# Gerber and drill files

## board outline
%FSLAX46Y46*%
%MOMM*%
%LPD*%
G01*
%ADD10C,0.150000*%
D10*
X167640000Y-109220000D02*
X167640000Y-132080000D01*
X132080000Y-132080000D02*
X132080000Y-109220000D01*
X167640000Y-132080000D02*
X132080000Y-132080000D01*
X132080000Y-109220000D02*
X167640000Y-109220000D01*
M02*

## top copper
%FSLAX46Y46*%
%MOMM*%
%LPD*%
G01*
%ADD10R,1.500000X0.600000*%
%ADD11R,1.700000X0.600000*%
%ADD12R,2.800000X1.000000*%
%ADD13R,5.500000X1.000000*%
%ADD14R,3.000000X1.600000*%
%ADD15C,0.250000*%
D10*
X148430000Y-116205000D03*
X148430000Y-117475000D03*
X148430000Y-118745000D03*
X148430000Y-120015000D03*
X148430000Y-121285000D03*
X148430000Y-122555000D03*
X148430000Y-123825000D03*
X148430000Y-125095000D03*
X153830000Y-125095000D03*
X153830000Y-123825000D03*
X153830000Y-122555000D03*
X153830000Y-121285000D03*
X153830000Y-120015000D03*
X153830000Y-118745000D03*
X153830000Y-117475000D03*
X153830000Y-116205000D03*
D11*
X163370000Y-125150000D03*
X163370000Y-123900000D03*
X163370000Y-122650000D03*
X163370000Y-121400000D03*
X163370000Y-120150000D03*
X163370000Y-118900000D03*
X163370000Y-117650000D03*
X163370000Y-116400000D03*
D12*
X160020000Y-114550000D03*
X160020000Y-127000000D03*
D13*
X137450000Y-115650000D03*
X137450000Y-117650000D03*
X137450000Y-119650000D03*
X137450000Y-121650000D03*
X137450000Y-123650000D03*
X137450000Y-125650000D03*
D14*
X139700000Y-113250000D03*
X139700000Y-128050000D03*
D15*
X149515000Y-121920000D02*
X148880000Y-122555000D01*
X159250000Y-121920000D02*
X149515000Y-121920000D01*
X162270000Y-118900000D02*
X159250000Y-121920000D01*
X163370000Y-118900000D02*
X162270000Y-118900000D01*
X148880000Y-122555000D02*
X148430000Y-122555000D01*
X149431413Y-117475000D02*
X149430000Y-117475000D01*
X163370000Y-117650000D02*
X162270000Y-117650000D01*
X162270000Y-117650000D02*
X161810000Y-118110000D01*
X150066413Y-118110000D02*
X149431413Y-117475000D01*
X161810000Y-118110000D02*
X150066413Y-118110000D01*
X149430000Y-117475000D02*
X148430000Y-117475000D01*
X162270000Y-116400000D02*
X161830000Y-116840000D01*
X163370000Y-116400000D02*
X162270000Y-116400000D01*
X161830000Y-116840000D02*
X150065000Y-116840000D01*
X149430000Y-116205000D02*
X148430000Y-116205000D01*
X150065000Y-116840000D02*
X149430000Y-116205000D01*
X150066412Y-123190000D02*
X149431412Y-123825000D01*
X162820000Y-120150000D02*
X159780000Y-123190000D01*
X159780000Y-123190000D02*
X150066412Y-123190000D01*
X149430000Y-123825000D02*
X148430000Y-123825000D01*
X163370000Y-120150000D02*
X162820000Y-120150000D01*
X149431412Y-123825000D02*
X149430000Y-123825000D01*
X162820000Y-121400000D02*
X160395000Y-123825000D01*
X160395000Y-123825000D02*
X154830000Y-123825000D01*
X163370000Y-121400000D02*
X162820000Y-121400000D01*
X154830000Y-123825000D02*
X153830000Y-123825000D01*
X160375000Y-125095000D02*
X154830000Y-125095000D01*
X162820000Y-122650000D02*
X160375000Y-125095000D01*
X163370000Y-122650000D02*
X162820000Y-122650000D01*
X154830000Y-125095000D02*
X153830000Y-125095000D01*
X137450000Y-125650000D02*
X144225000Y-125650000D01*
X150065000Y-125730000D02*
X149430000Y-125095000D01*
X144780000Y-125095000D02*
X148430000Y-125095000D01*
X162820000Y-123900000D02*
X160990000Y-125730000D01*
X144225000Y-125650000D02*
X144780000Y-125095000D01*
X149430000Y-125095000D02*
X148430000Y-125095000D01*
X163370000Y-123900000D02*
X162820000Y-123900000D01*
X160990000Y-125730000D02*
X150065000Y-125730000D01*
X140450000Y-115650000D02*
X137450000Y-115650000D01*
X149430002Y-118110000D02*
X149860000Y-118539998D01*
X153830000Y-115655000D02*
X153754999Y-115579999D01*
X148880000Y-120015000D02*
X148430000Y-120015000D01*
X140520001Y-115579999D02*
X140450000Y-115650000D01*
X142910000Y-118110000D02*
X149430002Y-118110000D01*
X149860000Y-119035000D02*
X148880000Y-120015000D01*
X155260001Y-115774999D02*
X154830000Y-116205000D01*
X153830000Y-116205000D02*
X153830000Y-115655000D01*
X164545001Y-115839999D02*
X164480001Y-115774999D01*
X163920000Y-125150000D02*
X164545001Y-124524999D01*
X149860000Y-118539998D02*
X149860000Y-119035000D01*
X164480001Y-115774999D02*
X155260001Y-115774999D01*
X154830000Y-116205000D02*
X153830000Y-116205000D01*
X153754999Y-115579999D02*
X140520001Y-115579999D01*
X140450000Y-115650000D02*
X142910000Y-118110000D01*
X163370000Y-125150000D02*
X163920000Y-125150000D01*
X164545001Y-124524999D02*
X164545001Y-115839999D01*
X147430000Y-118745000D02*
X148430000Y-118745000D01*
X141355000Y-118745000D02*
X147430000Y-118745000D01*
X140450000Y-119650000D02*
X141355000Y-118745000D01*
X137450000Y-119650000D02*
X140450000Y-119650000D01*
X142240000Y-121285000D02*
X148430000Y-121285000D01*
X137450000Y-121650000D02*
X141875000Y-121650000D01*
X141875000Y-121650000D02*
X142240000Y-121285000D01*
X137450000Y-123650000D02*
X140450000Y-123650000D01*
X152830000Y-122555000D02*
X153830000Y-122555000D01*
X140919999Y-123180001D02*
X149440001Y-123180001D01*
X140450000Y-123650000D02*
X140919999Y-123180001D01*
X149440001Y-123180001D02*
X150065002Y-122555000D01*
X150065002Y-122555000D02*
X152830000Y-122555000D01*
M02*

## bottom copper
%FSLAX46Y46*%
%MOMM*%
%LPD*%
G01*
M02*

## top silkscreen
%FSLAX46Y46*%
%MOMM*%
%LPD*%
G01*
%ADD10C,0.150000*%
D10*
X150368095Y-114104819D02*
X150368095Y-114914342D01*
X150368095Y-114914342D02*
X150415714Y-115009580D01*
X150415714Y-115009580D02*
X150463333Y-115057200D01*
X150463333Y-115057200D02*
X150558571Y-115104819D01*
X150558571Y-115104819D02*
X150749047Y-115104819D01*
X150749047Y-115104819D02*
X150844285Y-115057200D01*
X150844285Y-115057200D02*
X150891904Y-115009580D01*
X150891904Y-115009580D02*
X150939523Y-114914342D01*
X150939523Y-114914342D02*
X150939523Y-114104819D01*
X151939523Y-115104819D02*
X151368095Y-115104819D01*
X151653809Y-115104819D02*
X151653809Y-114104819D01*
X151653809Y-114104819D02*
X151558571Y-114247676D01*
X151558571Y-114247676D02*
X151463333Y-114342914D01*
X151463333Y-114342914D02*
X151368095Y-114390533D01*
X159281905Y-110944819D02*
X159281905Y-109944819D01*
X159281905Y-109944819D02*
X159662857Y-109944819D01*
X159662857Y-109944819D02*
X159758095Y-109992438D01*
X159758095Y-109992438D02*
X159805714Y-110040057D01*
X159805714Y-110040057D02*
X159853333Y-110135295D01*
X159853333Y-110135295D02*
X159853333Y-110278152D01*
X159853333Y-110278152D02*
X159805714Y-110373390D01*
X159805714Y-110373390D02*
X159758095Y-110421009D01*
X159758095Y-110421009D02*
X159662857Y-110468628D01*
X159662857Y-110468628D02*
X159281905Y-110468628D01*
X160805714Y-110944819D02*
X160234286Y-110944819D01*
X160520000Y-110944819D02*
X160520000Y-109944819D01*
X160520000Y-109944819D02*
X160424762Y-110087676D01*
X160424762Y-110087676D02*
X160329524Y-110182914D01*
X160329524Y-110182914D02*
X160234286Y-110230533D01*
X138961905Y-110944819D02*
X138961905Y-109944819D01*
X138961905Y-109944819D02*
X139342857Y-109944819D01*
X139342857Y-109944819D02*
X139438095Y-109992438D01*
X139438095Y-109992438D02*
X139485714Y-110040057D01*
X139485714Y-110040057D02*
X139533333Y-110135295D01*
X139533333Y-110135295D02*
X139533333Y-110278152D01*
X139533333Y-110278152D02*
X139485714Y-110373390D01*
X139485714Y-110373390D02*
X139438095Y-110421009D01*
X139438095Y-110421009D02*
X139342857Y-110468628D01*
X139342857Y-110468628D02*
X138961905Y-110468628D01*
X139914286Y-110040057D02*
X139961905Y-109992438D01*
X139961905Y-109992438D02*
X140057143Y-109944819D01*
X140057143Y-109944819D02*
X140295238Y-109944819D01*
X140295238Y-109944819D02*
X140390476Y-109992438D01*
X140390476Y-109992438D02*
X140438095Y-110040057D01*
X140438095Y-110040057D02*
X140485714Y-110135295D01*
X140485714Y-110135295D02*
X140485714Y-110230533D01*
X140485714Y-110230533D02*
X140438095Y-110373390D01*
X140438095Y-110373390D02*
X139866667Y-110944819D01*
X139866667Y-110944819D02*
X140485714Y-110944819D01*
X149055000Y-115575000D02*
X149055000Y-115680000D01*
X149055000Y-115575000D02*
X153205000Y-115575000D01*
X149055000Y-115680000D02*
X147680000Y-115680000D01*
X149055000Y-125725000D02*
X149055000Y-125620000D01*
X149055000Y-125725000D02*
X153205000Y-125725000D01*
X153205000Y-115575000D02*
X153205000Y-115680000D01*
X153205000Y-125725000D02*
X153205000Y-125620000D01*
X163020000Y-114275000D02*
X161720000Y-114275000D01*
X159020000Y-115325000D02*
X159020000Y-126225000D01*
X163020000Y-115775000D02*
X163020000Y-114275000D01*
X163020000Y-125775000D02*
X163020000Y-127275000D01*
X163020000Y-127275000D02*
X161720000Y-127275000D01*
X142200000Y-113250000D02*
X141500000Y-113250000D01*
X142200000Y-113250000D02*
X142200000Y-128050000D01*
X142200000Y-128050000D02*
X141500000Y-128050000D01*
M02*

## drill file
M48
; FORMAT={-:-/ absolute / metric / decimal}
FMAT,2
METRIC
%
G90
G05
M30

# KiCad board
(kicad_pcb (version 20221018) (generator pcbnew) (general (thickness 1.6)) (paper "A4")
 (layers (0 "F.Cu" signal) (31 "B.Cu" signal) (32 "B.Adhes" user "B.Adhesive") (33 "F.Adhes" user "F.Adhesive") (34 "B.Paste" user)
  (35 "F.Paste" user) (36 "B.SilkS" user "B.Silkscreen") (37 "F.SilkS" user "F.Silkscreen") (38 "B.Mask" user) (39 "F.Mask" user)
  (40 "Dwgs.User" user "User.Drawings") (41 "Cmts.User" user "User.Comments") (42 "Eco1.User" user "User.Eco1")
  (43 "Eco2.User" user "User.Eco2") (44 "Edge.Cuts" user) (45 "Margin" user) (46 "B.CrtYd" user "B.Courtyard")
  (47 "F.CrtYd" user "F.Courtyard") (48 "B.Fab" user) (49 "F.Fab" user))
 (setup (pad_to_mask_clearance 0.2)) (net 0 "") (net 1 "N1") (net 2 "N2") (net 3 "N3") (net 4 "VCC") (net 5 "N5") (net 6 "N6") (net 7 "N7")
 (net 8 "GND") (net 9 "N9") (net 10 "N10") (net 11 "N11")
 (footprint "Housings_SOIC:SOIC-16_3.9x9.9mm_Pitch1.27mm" (layer "F.Cu") (at 151.13 120.65)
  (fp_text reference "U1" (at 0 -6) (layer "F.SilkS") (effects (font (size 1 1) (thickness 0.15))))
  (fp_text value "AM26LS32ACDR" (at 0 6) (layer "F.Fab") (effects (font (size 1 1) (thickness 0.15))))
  (fp_line (start -2.075 -5.075) (end -2.075 -4.97) (stroke (width 0.15) (type solid)) (layer "F.SilkS"))
  (fp_line (start -2.075 -5.075) (end 2.075 -5.075) (stroke (width 0.15) (type solid)) (layer "F.SilkS"))
  (fp_line (start -2.075 -4.97) (end -3.45 -4.97) (stroke (width 0.15) (type solid)) (layer "F.SilkS"))
  (fp_line (start -2.075 5.075) (end -2.075 4.97) (stroke (width 0.15) (type solid)) (layer "F.SilkS"))
  (fp_line (start -2.075 5.075) (end 2.075 5.075) (stroke (width 0.15) (type solid)) (layer "F.SilkS"))
  (fp_line (start 2.075 -5.075) (end 2.075 -4.97) (stroke (width 0.15) (type solid)) (layer "F.SilkS"))
  (fp_line (start 2.075 5.075) (end 2.075 4.97) (stroke (width 0.15) (type solid)) (layer "F.SilkS"))
  (pad "1" smd rect (at -2.7 -4.445) (size 1.5 0.6) (layers "F.Cu" "F.Paste" "F.Mask") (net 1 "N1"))
  (pad "2" smd rect (at -2.7 -3.175) (size 1.5 0.6) (layers "F.Cu" "F.Paste" "F.Mask") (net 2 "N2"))
  (pad "3" smd rect (at -2.7 -1.905) (size 1.5 0.6) (layers "F.Cu" "F.Paste" "F.Mask") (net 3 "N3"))
  (pad "4" smd rect (at -2.7 -0.635) (size 1.5 0.6) (layers "F.Cu" "F.Paste" "F.Mask") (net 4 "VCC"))
  (pad "5" smd rect (at -2.7 0.635) (size 1.5 0.6) (layers "F.Cu" "F.Paste" "F.Mask") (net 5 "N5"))
  (pad "6" smd rect (at -2.7 1.905) (size 1.5 0.6) (layers "F.Cu" "F.Paste" "F.Mask") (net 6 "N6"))
  (pad "7" smd rect (at -2.7 3.175) (size 1.5 0.6) (layers "F.Cu" "F.Paste" "F.Mask") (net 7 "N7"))
  (pad "8" smd rect (at -2.7 4.445) (size 1.5 0.6) (layers "F.Cu" "F.Paste" "F.Mask") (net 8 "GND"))
  (pad "9" smd rect (at 2.7 4.445) (size 1.5 0.6) (layers "F.Cu" "F.Paste" "F.Mask") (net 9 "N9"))
  (pad "10" smd rect (at 2.7 3.175) (size 1.5 0.6) (layers "F.Cu" "F.Paste" "F.Mask") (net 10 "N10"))
  (pad "11" smd rect (at 2.7 1.905) (size 1.5 0.6) (layers "F.Cu" "F.Paste" "F.Mask") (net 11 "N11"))
  (pad "12" smd rect (at 2.7 0.635) (size 1.5 0.6) (layers "F.Cu" "F.Paste" "F.Mask"))
  (pad "13" smd rect (at 2.7 -0.635) (size 1.5 0.6) (layers "F.Cu" "F.Paste" "F.Mask"))
  (pad "14" smd rect (at 2.7 -1.905) (size 1.5 0.6) (layers "F.Cu" "F.Paste" "F.Mask"))
  (pad "15" smd rect (at 2.7 -3.175) (size 1.5 0.6) (layers "F.Cu" "F.Paste" "F.Mask"))
  (pad "16" smd rect (at 2.7 -4.445) (size 1.5 0.6) (layers "F.Cu" "F.Paste" "F.Mask") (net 4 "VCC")))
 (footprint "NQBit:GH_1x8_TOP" (layer "F.Cu") (at 160.02 120.775 -90)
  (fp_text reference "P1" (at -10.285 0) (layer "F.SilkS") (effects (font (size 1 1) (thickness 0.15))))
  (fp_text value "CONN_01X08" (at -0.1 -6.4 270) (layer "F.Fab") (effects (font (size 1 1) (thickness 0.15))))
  (fp_line (start -6.5 -3) (end -6.5 -1.7) (stroke (width 0.15) (type solid)) (layer "F.SilkS"))
  (fp_line (start -5.45 1) (end 5.45 1) (stroke (width 0.15) (type solid)) (layer "F.SilkS"))
  (fp_line (start -5 -3) (end -6.5 -3) (stroke (width 0.15) (type solid)) (layer "F.SilkS"))
  (fp_line (start 5 -3) (end 6.5 -3) (stroke (width 0.15) (type solid)) (layer "F.SilkS"))
  (fp_line (start 6.5 -3) (end 6.5 -1.7) (stroke (width 0.15) (type solid)) (layer "F.SilkS"))
  (pad "1" smd rect (at 4.375 -3.35 270) (size 0.6 1.7) (layers "F.Cu" "F.Paste" "F.Mask") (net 4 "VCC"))
  (pad "2" smd rect (at 3.125 -3.35 270) (size 0.6 1.7) (layers "F.Cu" "F.Paste" "F.Mask") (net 8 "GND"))
  (pad "3" smd rect (at 1.875 -3.35 270) (size 0.6 1.7) (layers "F.Cu" "F.Paste" "F.Mask") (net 9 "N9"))
  (pad "4" smd rect (at 0.625 -3.35 270) (size 0.6 1.7) (layers "F.Cu" "F.Paste" "F.Mask") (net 10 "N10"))
  (pad "5" smd rect (at -0.625 -3.35 270) (size 0.6 1.7) (layers "F.Cu" "F.Paste" "F.Mask") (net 7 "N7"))
  (pad "6" smd rect (at -1.875 -3.35 270) (size 0.6 1.7) (layers "F.Cu" "F.Paste" "F.Mask") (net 6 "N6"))
  (pad "7" smd rect (at -3.125 -3.35 270) (size 0.6 1.7) (layers "F.Cu" "F.Paste" "F.Mask") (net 2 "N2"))
  (pad "8" smd rect (at -4.375 -3.35 270) (size 0.6 1.7) (layers "F.Cu" "F.Paste" "F.Mask") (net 1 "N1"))
  (pad "MECH" smd rect (at -6.225 0 270) (size 1 2.8) (layers "F.Cu" "F.Paste" "F.Mask"))
  (pad "MECH" smd rect (at 6.225 0 270) (size 1 2.8) (layers "F.Cu" "F.Paste" "F.Mask")))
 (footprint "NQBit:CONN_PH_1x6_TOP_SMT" (layer "F.Cu") (at 139.7 120.65 -90)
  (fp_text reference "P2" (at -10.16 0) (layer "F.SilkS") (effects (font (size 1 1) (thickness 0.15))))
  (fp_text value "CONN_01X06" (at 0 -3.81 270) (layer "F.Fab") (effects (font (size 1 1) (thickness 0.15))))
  (fp_line (start -7.4 -2.5) (end -7.4 -1.8) (stroke (width 0.15) (type solid)) (layer "F.SilkS"))
  (fp_line (start -7.4 -2.5) (end 7.4 -2.5) (stroke (width 0.15) (type solid)) (layer "F.SilkS"))
  (fp_line (start 7.4 -2.5) (end 7.4 -1.8) (stroke (width 0.15) (type solid)) (layer "F.SilkS"))
  (pad "1" smd rect (at -5 2.25 270) (size 1 5.5) (layers "F.Cu" "F.Paste" "F.Mask") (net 4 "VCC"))
  (pad "2" smd rect (at -3 2.25 270) (size 1 5.5) (layers "F.Cu" "F.Paste" "F.Mask"))
  (pad "3" smd rect (at -1 2.25 270) (size 1 5.5) (layers "F.Cu" "F.Paste" "F.Mask") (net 3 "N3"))
  (pad "4" smd rect (at 1 2.25 270) (size 1 5.5) (layers "F.Cu" "F.Paste" "F.Mask") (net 5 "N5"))
  (pad "5" smd rect (at 3 2.25 270) (size 1 5.5) (layers "F.Cu" "F.Paste" "F.Mask") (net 11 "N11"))
  (pad "6" smd rect (at 5 2.25 270) (size 1 5.5) (layers "F.Cu" "F.Paste" "F.Mask") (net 8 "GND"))
  (pad "MECH" smd rect (at -7.4 0 270) (size 1.6 3) (layers "F.Cu" "F.Paste" "F.Mask"))
  (pad "MECH" smd rect (at 7.4 0 270) (size 1.6 3) (layers "F.Cu" "F.Paste" "F.Mask")))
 (gr_line (start 167.64 109.22) (end 167.64 132.08) (stroke (width 0.15) (type solid)) (layer "Edge.Cuts"))
 (gr_line (start 132.08 132.08) (end 132.08 109.22) (stroke (width 0.15) (type solid)) (layer "Edge.Cuts"))
 (gr_line (start 167.64 132.08) (end 132.08 132.08) (stroke (width 0.15) (type solid)) (layer "Edge.Cuts"))
 (gr_line (start 132.08 109.22) (end 167.64 109.22) (stroke (width 0.15) (type solid)) (layer "Edge.Cuts"))
 (segment (start 149.515 121.92) (end 148.88 122.555) (width 0.25) (layer "F.Cu") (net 6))
 (segment (start 159.25 121.92) (end 149.515 121.92) (width 0.25) (layer "F.Cu") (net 6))
 (segment (start 162.27 118.9) (end 159.25 121.92) (width 0.25) (layer "F.Cu") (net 6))
 (segment (start 163.37 118.9) (end 162.27 118.9) (width 0.25) (layer "F.Cu") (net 6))
 (segment (start 148.88 122.555) (end 148.43 122.555) (width 0.25) (layer "F.Cu") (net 6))
 (segment (start 149.431413 117.475) (end 149.43 117.475) (width 0.25) (layer "F.Cu") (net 2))
 (segment (start 163.37 117.65) (end 162.27 117.65) (width 0.25) (layer "F.Cu") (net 2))
 (segment (start 162.27 117.65) (end 161.81 118.11) (width 0.25) (layer "F.Cu") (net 2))
 (segment (start 150.066413 118.11) (end 149.431413 117.475) (width 0.25) (layer "F.Cu") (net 2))
 (segment (start 161.81 118.11) (end 150.066413 118.11) (width 0.25) (layer "F.Cu") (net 2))
 (segment (start 149.43 117.475) (end 148.43 117.475) (width 0.25) (layer "F.Cu") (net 2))
 (segment (start 162.27 116.4) (end 161.83 116.84) (width 0.25) (layer "F.Cu") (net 1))
 (segment (start 163.37 116.4) (end 162.27 116.4) (width 0.25) (layer "F.Cu") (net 1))
 (segment (start 161.83 116.84) (end 150.065 116.84) (width 0.25) (layer "F.Cu") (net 1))
 (segment (start 149.43 116.205) (end 148.43 116.205) (width 0.25) (layer "F.Cu") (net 1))
 (segment (start 150.065 116.84) (end 149.43 116.205) (width 0.25) (layer "F.Cu") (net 1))
 (segment (start 150.066412 123.19) (end 149.431412 123.825) (width 0.25) (layer "F.Cu") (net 7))
 (segment (start 162.82 120.15) (end 159.78 123.19) (width 0.25) (layer "F.Cu") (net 7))
 (segment (start 159.78 123.19) (end 150.066412 123.19) (width 0.25) (layer "F.Cu") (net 7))
 (segment (start 149.43 123.825) (end 148.43 123.825) (width 0.25) (layer "F.Cu") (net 7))
 (segment (start 163.37 120.15) (end 162.82 120.15) (width 0.25) (layer "F.Cu") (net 7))
 (segment (start 149.431412 123.825) (end 149.43 123.825) (width 0.25) (layer "F.Cu") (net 7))
 (segment (start 162.82 121.4) (end 160.395 123.825) (width 0.25) (layer "F.Cu") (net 10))
 (segment (start 160.395 123.825) (end 154.83 123.825) (width 0.25) (layer "F.Cu") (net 10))
 (segment (start 163.37 121.4) (end 162.82 121.4) (width 0.25) (layer "F.Cu") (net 10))
 (segment (start 154.83 123.825) (end 153.83 123.825) (width 0.25) (layer "F.Cu") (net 10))
 (segment (start 160.375 125.095) (end 154.83 125.095) (width 0.25) (layer "F.Cu") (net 9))
 (segment (start 162.82 122.65) (end 160.375 125.095) (width 0.25) (layer "F.Cu") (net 9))
 (segment (start 163.37 122.65) (end 162.82 122.65) (width 0.25) (layer "F.Cu") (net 9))
 (segment (start 154.83 125.095) (end 153.83 125.095) (width 0.25) (layer "F.Cu") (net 9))
 (segment (start 137.45 125.65) (end 144.225 125.65) (width 0.25) (layer "F.Cu") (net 8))
 (segment (start 150.065 125.73) (end 149.43 125.095) (width 0.25) (layer "F.Cu") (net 8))
 (segment (start 144.78 125.095) (end 148.43 125.095) (width 0.25) (layer "F.Cu") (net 8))
 (segment (start 162.82 123.9) (end 160.99 125.73) (width 0.25) (layer "F.Cu") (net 8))
 (segment (start 144.225 125.65) (end 144.78 125.095) (width 0.25) (layer "F.Cu") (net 8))
 (segment (start 149.43 125.095) (end 148.43 125.095) (width 0.25) (layer "F.Cu") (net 8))
 (segment (start 163.37 123.9) (end 162.82 123.9) (width 0.25) (layer "F.Cu") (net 8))
 (segment (start 160.99 125.73) (end 150.065 125.73) (width 0.25) (layer "F.Cu") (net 8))
 (segment (start 140.45 115.65) (end 137.45 115.65) (width 0.25) (layer "F.Cu") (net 4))
 (segment (start 149.430002 118.11) (end 149.86 118.539998) (width 0.25) (layer "F.Cu") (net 4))
 (segment (start 153.83 115.655) (end 153.754999 115.579999) (width 0.25) (layer "F.Cu") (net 4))
 (segment (start 148.88 120.015) (end 148.43 120.015) (width 0.25) (layer "F.Cu") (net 4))
 (segment (start 140.520001 115.579999) (end 140.45 115.65) (width 0.25) (layer "F.Cu") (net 4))
 (segment (start 142.91 118.11) (end 149.430002 118.11) (width 0.25) (layer "F.Cu") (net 4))
 (segment (start 149.86 119.035) (end 148.88 120.015) (width 0.25) (layer "F.Cu") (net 4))
 (segment (start 155.260001 115.774999) (end 154.83 116.205) (width 0.25) (layer "F.Cu") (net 4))
 (segment (start 153.83 116.205) (end 153.83 115.655) (width 0.25) (layer "F.Cu") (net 4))
 (segment (start 164.545001 115.839999) (end 164.480001 115.774999) (width 0.25) (layer "F.Cu") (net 4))
 (segment (start 163.92 125.15) (end 164.545001 124.524999) (width 0.25) (layer "F.Cu") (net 4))
 (segment (start 149.86 118.539998) (end 149.86 119.035) (width 0.25) (layer "F.Cu") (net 4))
 (segment (start 164.480001 115.774999) (end 155.260001 115.774999) (width 0.25) (layer "F.Cu") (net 4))
 (segment (start 154.83 116.205) (end 153.83 116.205) (width 0.25) (layer "F.Cu") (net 4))
 (segment (start 153.754999 115.579999) (end 140.520001 115.579999) (width 0.25) (layer "F.Cu") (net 4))
 (segment (start 140.45 115.65) (end 142.91 118.11) (width 0.25) (layer "F.Cu") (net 4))
 (segment (start 163.37 125.15) (end 163.92 125.15) (width 0.25) (layer "F.Cu") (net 4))
 (segment (start 164.545001 124.524999) (end 164.545001 115.839999) (width 0.25) (layer "F.Cu") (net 4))
 (segment (start 147.43 118.745) (end 148.43 118.745) (width 0.25) (layer "F.Cu") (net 3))
 (segment (start 141.355 118.745) (end 147.43 118.745) (width 0.25) (layer "F.Cu") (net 3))
 (segment (start 140.45 119.65) (end 141.355 118.745) (width 0.25) (layer "F.Cu") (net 3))
 (segment (start 137.45 119.65) (end 140.45 119.65) (width 0.25) (layer "F.Cu") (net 3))
 (segment (start 142.24 121.285) (end 148.43 121.285) (width 0.25) (layer "F.Cu") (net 5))
 (segment (start 137.45 121.65) (end 141.875 121.65) (width 0.25) (layer "F.Cu") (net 5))
 (segment (start 141.875 121.65) (end 142.24 121.285) (width 0.25) (layer "F.Cu") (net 5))
 (segment (start 137.45 123.65) (end 140.45 123.65) (width 0.25) (layer "F.Cu") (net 11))
 (segment (start 152.83 122.555) (end 153.83 122.555) (width 0.25) (layer "F.Cu") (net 11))
 (segment (start 140.919999 123.180001) (end 149.440001 123.180001) (width 0.25) (layer "F.Cu") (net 11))
 (segment (start 140.45 123.65) (end 140.919999 123.180001) (width 0.25) (layer "F.Cu") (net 11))
 (segment (start 149.440001 123.180001) (end 150.065002 122.555) (width 0.25) (layer "F.Cu") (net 11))
 (segment (start 150.065002 122.555) (end 152.83 122.555) (width 0.25) (layer "F.Cu") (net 11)))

